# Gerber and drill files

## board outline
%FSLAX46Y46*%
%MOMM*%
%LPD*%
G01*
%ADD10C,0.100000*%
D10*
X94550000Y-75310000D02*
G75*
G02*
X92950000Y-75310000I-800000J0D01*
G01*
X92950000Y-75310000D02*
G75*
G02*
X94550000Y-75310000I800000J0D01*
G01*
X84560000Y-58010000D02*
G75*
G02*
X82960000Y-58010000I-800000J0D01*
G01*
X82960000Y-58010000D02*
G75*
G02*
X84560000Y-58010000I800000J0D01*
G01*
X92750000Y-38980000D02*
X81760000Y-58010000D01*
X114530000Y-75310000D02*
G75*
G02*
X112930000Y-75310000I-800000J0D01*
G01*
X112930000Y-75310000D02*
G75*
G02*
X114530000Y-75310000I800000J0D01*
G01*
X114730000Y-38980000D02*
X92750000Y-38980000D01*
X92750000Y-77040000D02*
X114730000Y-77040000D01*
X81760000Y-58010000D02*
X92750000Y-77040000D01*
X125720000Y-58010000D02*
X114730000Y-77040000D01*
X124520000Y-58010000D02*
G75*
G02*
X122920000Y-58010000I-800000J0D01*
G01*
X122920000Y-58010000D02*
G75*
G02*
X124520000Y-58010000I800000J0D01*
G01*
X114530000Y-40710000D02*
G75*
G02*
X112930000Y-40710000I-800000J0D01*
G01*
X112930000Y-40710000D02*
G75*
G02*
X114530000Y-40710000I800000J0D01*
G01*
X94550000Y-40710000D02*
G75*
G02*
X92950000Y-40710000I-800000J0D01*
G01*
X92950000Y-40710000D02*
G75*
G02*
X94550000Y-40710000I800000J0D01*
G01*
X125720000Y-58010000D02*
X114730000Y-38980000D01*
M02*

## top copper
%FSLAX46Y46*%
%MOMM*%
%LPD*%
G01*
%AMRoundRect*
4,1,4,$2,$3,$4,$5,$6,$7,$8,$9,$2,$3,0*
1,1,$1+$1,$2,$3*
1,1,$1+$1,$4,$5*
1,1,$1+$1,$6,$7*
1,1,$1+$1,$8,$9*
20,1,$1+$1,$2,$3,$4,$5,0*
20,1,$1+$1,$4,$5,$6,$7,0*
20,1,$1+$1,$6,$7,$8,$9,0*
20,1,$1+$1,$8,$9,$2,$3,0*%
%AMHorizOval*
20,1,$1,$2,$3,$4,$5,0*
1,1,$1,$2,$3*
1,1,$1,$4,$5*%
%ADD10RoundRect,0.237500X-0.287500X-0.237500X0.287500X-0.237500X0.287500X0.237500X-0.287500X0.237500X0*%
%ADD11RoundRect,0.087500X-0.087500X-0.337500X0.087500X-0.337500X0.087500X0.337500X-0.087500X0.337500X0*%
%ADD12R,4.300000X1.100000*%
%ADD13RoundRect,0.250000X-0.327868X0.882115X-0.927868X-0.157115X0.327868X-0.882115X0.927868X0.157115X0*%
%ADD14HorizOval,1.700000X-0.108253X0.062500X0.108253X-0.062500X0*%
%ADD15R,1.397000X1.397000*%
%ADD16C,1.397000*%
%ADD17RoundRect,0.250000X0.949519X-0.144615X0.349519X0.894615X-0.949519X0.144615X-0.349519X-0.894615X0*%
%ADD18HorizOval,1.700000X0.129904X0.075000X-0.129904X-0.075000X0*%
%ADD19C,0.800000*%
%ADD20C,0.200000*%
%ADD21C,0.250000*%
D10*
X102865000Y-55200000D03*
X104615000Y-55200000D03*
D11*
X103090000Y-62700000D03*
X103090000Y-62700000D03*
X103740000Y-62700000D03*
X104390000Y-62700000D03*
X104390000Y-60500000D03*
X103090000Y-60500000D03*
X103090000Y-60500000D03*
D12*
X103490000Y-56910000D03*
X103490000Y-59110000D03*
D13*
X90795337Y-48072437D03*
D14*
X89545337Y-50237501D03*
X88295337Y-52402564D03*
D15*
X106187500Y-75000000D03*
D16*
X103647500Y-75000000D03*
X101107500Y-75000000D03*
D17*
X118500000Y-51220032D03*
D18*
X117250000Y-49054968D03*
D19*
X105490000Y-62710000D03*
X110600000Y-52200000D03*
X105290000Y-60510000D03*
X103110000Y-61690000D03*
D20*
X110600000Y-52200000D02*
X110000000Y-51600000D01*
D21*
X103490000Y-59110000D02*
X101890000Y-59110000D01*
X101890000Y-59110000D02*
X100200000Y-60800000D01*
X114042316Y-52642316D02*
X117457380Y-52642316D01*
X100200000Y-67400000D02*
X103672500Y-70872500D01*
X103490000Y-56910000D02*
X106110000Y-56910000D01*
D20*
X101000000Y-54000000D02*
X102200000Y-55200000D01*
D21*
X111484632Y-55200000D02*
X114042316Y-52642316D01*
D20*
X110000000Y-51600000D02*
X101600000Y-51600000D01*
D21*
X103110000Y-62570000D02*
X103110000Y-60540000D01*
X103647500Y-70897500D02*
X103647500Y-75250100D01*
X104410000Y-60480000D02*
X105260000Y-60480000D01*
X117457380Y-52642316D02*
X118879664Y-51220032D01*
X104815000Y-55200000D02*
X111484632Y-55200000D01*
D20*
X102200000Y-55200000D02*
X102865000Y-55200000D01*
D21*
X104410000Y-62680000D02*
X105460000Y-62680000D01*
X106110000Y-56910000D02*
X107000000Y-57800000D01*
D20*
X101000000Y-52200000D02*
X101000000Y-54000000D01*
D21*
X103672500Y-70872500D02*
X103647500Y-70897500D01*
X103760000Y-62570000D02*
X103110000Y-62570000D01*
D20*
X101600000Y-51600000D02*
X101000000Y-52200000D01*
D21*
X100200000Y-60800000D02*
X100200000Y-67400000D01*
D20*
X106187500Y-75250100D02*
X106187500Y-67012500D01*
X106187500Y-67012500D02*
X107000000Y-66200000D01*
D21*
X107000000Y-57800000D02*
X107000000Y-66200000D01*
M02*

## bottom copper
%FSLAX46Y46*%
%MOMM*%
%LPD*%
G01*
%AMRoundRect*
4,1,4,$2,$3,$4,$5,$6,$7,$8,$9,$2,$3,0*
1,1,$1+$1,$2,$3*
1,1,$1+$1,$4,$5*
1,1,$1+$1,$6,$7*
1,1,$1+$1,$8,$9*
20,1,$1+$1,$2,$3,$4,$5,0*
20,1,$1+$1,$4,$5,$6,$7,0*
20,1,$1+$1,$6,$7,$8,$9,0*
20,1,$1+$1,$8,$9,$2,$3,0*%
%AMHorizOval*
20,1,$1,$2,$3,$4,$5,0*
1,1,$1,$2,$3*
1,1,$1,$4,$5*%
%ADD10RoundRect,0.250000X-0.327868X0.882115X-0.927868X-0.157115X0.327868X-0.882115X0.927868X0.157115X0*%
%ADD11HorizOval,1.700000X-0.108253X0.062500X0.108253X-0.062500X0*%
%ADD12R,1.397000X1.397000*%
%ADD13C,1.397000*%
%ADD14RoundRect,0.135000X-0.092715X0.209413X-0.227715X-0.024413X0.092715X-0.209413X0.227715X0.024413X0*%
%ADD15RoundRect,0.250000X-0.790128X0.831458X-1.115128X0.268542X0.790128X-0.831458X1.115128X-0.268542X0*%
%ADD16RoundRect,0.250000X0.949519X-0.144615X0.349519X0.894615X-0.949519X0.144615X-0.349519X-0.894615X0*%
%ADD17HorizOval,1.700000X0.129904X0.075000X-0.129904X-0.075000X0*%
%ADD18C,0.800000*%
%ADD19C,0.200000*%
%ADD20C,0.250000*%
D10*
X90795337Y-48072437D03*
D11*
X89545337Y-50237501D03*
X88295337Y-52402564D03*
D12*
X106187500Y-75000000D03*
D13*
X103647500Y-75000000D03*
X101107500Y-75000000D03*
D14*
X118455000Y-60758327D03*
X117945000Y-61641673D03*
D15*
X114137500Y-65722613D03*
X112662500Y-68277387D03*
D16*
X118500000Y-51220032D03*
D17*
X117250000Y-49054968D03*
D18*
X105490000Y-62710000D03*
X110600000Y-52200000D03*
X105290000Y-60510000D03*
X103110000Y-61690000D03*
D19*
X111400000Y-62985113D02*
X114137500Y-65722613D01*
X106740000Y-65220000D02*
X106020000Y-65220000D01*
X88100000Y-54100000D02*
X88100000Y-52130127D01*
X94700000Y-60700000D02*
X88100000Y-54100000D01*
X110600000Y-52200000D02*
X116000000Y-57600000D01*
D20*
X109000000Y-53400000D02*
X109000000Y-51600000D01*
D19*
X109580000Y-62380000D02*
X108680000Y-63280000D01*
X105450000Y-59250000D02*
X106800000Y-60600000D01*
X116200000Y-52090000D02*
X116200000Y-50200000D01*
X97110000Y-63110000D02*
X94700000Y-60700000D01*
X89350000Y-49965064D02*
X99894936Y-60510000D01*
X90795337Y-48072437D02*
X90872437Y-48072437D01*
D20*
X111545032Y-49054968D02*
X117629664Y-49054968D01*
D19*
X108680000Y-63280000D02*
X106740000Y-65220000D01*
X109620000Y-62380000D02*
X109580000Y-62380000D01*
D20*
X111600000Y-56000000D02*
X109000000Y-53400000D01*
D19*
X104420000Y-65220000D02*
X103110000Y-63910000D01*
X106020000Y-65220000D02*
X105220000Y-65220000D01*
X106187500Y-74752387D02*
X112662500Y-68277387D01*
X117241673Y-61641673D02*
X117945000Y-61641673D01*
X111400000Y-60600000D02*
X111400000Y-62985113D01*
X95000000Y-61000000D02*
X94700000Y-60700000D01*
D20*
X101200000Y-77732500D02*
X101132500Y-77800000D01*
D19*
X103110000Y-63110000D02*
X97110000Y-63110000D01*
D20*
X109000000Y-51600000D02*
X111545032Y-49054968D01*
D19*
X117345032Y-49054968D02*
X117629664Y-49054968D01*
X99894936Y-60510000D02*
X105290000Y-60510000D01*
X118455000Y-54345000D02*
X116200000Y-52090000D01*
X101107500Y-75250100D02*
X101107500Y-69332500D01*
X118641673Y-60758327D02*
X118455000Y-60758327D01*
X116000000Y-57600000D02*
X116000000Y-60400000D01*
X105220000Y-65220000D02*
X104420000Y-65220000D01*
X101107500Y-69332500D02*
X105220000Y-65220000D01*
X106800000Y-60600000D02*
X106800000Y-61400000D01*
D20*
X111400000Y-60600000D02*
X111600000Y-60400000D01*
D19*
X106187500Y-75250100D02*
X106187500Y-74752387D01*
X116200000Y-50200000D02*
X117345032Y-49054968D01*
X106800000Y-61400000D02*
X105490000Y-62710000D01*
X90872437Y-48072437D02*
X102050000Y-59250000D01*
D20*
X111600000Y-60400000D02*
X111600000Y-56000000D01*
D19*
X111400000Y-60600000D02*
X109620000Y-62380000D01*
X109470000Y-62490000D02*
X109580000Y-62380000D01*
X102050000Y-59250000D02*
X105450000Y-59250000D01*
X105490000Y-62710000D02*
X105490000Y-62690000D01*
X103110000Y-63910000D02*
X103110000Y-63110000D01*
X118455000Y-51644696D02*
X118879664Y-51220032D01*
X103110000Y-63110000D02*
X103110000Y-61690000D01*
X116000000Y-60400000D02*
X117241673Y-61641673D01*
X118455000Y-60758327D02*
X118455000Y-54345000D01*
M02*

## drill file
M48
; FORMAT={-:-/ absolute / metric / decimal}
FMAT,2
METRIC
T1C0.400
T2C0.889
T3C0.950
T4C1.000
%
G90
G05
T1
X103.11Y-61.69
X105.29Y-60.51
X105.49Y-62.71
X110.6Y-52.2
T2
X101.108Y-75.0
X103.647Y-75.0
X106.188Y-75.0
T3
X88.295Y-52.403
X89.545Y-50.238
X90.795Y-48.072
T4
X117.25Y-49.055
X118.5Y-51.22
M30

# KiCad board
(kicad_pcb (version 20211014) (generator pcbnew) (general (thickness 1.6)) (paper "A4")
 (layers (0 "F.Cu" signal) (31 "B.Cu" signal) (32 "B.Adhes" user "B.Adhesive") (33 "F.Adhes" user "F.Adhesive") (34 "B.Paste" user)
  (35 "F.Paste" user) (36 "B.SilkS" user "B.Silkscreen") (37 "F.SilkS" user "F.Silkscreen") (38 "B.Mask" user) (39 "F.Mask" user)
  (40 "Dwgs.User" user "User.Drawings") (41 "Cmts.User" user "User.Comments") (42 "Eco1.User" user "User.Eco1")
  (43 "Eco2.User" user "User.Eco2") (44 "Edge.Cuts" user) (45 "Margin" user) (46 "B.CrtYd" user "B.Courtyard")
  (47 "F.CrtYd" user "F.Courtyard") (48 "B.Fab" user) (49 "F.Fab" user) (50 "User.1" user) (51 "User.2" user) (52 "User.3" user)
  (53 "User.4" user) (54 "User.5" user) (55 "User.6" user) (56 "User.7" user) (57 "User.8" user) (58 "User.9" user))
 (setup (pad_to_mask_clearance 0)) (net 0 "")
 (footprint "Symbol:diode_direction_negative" (layer "F.Cu") (at 103.8 52.65)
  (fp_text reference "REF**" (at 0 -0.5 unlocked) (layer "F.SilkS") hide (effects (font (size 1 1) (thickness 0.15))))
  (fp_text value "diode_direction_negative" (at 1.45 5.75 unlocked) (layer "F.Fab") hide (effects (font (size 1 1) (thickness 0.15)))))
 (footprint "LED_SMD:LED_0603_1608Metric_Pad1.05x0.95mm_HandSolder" (layer "F.Cu") (at 103.74 55.2)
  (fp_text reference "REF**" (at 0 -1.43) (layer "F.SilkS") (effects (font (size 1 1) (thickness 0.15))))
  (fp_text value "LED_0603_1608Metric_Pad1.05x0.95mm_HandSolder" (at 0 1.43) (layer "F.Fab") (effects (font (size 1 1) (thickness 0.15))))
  (pad "1" smd roundrect (at -0.875 0) (size 1.05 0.95) (layers "F.Cu" "F.Paste" "F.Mask") (roundrect_rratio 0.25))
  (pad "2" smd roundrect (at 0.875 0) (size 1.05 0.95) (layers "F.Cu" "F.Paste" "F.Mask") (roundrect_rratio 0.25)))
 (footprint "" (layer "F.Cu") (at 103.09 62.7)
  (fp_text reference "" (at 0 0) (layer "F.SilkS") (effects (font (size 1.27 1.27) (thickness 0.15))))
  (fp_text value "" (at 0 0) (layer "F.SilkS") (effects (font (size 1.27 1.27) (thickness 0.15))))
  (pad "1" smd roundrect (at 0 0) (size 0.35 0.85) (layers "F.Cu" "F.Paste" "F.Mask") (roundrect_rratio 0.25)))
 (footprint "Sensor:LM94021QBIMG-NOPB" (layer "F.Cu") (at 103.74 61.6)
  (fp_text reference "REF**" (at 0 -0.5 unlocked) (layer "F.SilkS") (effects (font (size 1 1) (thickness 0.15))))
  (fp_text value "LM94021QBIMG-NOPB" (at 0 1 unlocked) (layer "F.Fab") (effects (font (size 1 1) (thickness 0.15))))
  (pad "1" smd roundrect (at -0.65 1.1) (size 0.35 0.85) (layers "F.Cu" "F.Paste" "F.Mask") (roundrect_rratio 0.25))
  (pad "2" smd roundrect (at 0 1.1) (size 0.35 0.85) (layers "F.Cu" "F.Paste" "F.Mask") (roundrect_rratio 0.25))
  (pad "3" smd roundrect (at 0.65 1.1) (size 0.35 0.85) (layers "F.Cu" "F.Paste" "F.Mask") (roundrect_rratio 0.25))
  (pad "4" smd roundrect (at 0.65 -1.1) (size 0.35 0.85) (layers "F.Cu" "F.Paste" "F.Mask") (roundrect_rratio 0.25))
  (pad "5" smd roundrect (at -0.65 -1.1) (size 0.35 0.85) (layers "F.Cu" "F.Paste" "F.Mask") (roundrect_rratio 0.25)))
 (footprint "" (layer "F.Cu") (at 103.09 60.5)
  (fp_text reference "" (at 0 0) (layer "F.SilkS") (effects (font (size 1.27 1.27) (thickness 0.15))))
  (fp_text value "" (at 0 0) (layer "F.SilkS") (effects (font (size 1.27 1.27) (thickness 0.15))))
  (pad "5" smd roundrect (at 0 0) (size 0.35 0.85) (layers "F.Cu" "F.Paste" "F.Mask") (roundrect_rratio 0.25)))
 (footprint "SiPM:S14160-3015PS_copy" (layer "F.Cu") (at 103.74 58.01)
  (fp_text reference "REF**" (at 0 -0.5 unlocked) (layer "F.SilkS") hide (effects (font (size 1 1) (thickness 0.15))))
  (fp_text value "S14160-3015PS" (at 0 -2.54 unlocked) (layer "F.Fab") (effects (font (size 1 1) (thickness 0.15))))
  (pad "1" smd rect (at -0.25 -1.1) (size 4.3 1.1) (layers "F.Cu" "F.Paste" "F.Mask"))
  (pad "2" smd rect (at -0.25 1.1) (size 4.3 1.1) (layers "F.Cu" "F.Paste" "F.Mask")))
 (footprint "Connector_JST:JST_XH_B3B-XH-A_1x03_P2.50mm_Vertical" (layer "B.Cu") (at 90.795337 48.072437 -120)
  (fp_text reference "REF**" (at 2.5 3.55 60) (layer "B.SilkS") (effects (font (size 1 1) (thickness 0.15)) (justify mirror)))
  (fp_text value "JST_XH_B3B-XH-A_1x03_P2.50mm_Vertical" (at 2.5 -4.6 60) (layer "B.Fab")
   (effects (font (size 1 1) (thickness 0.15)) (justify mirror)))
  (pad "1" thru_hole roundrect (at 0 0 240) (size 1.7 1.95) (drill 0.95) (layers *.Cu *.Mask) (roundrect_rratio 0.1470588235))
  (pad "2" thru_hole oval (at 2.5 0 240) (size 1.7 1.95) (drill 0.95) (layers *.Cu *.Mask))
  (pad "3" thru_hole oval (at 5 0 240) (size 1.7 1.95) (drill 0.95) (layers *.Cu *.Mask)))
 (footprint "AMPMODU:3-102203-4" (layer "B.Cu") (at 106.1875 75 180)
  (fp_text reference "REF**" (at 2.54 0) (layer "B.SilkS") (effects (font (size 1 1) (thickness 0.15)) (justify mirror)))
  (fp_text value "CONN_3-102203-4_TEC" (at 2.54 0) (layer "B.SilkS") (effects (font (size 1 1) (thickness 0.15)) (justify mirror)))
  (pad "1" thru_hole rect locked (at 0 0 180) (size 1.397 1.397) (drill 0.889) (layers *.Cu *.Mask))
  (pad "2" thru_hole circle locked (at 2.54 0 180) (size 1.397 1.397) (drill 0.889) (layers *.Cu *.Mask))
  (pad "3" thru_hole circle locked (at 5.08 0 180) (size 1.397 1.397) (drill 0.889) (layers *.Cu *.Mask)))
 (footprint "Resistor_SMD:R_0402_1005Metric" (layer "B.Cu") (at 118.2 61.2 -120)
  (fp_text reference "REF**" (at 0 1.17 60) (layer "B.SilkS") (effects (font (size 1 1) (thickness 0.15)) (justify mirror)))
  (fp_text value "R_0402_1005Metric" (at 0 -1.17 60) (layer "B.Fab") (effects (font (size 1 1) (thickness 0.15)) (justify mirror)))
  (pad "1" smd roundrect (at -0.51 0 240) (size 0.54 0.64) (layers "B.Cu" "B.Paste" "B.Mask") (roundrect_rratio 0.25))
  (pad "2" smd roundrect (at 0.51 0 240) (size 0.54 0.64) (layers "B.Cu" "B.Paste" "B.Mask") (roundrect_rratio 0.25)))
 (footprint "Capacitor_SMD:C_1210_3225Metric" (layer "B.Cu") (at 113.4 67 -120)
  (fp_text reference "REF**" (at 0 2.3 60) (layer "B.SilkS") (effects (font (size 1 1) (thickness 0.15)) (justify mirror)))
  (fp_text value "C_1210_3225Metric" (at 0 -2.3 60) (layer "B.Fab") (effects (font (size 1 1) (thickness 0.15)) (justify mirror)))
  (pad "1" smd roundrect (at -1.475 0 240) (size 1.15 2.7) (layers "B.Cu" "B.Paste" "B.Mask") (roundrect_rratio 0.2173913043))
  (pad "2" smd roundrect (at 1.475 0 240) (size 1.15 2.7) (layers "B.Cu" "B.Paste" "B.Mask") (roundrect_rratio 0.2173913043)))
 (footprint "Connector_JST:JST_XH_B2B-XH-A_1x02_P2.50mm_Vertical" (layer "B.Cu") (at 118.5 51.220032 120)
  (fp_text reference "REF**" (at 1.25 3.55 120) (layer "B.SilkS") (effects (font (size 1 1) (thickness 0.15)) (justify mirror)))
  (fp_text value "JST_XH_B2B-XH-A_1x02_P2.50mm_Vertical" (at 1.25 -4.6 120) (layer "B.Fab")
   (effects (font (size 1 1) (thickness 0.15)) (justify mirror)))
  (pad "1" thru_hole roundrect (at 0 0 120) (size 1.7 2) (drill 1) (layers *.Cu *.Mask) (roundrect_rratio 0.1470588235))
  (pad "2" thru_hole oval (at 2.5 0 120) (size 1.7 2) (drill 1) (layers *.Cu *.Mask)))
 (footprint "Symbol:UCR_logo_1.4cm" (layer "B.Cu") (at 104.4 43 180)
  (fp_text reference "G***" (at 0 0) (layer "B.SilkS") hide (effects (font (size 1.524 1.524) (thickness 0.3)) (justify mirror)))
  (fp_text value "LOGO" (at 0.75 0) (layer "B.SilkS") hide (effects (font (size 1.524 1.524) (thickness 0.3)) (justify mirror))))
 (gr_circle (center 93.75 75.31) (end 94.55 75.31) (layer "Edge.Cuts") (width 0.1) (fill none))
 (gr_circle (center 83.76 58.01) (end 84.56 58.01) (layer "Edge.Cuts") (width 0.1) (fill none))
 (gr_line (start 92.75 38.98) (end 81.76 58.01) (layer "Edge.Cuts") (width 0.1))
 (gr_circle (center 113.73 75.31) (end 114.53 75.31) (layer "Edge.Cuts") (width 0.1) (fill none))
 (gr_line (start 114.73 38.98) (end 92.75 38.98) (layer "Edge.Cuts") (width 0.1))
 (gr_line (start 92.75 77.04) (end 114.73 77.04) (layer "Edge.Cuts") (width 0.1))
 (gr_line (start 81.76 58.01) (end 92.75 77.04) (layer "Edge.Cuts") (width 0.1))
 (gr_line (start 125.72 58.01) (end 114.73 77.04) (layer "Edge.Cuts") (width 0.1))
 (gr_circle (center 123.72 58.01) (end 124.52 58.01) (layer "Edge.Cuts") (width 0.1) (fill none))
 (gr_circle (center 113.73 40.71) (end 114.53 40.71) (layer "Edge.Cuts") (width 0.1) (fill none))
 (gr_circle (center 93.75 40.71) (end 94.55 40.71) (layer "Edge.Cuts") (width 0.1) (fill none))
 (gr_line (start 125.72 58.01) (end 114.73 38.98) (layer "Edge.Cuts") (width 0.1))
 (segment (start 110.6 52.2) (end 110 51.6) (width 0.2) (layer "F.Cu") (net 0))
 (segment (start 103.49 59.11) (end 101.89 59.11) (width 0.25) (layer "F.Cu") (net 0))
 (segment (start 101.89 59.11) (end 100.2 60.8) (width 0.25) (layer "F.Cu") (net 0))
 (segment (start 114.042316 52.642316) (end 117.45738 52.642316) (width 0.25) (layer "F.Cu") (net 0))
 (segment (start 100.2 67.4) (end 103.6725 70.8725) (width 0.25) (layer "F.Cu") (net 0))
 (segment (start 103.49 56.91) (end 106.11 56.91) (width 0.25) (layer "F.Cu") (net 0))
 (segment (start 101 54) (end 102.2 55.2) (width 0.2) (layer "F.Cu") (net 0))
 (segment (start 111.484632 55.2) (end 114.042316 52.642316) (width 0.25) (layer "F.Cu") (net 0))
 (segment (start 110 51.6) (end 101.6 51.6) (width 0.2) (layer "F.Cu") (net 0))
 (segment (start 103.11 62.57) (end 103.11 60.54) (width 0.25) (layer "F.Cu") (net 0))
 (segment (start 103.6475 70.8975) (end 103.6475 75.2501) (width 0.25) (layer "F.Cu") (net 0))
 (segment (start 104.41 60.48) (end 105.26 60.48) (width 0.25) (layer "F.Cu") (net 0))
 (segment (start 117.45738 52.642316) (end 118.879664 51.220032) (width 0.25) (layer "F.Cu") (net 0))
 (segment (start 104.815 55.2) (end 111.484632 55.2) (width 0.25) (layer "F.Cu") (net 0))
 (segment (start 102.2 55.2) (end 102.865 55.2) (width 0.2) (layer "F.Cu") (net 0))
 (segment (start 104.41 62.68) (end 105.46 62.68) (width 0.25) (layer "F.Cu") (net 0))
 (segment (start 106.11 56.91) (end 107 57.8) (width 0.25) (layer "F.Cu") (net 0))
 (segment (start 101 52.2) (end 101 54) (width 0.2) (layer "F.Cu") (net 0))
 (segment (start 103.6725 70.8725) (end 103.6475 70.8975) (width 0.25) (layer "F.Cu") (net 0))
 (segment (start 103.76 62.57) (end 103.11 62.57) (width 0.25) (layer "F.Cu") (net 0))
 (segment (start 101.6 51.6) (end 101 52.2) (width 0.2) (layer "F.Cu") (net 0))
 (segment (start 100.2 60.8) (end 100.2 67.4) (width 0.25) (layer "F.Cu") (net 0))
 (segment (start 106.1875 75.2501) (end 106.1875 67.0125) (width 0.2) (layer "F.Cu") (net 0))
 (segment (start 106.1875 67.0125) (end 107 66.2) (width 0.2) (layer "F.Cu") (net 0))
 (segment (start 107 57.8) (end 107 66.2) (width 0.25) (layer "F.Cu") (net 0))
 (via (at 105.49 62.71) (size 0.8) (drill 0.4) (layers "F.Cu" "B.Cu") (free) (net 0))
 (via (at 110.6 52.2) (size 0.8) (drill 0.4) (layers "F.Cu" "B.Cu") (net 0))
 (via (at 105.29 60.51) (size 0.8) (drill 0.4) (layers "F.Cu" "B.Cu") (free) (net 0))
 (via (at 103.11 61.69) (size 0.8) (drill 0.4) (layers "F.Cu" "B.Cu") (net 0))
 (segment (start 111.4 62.985113) (end 114.1375 65.722613) (width 0.2) (layer "B.Cu") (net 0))
 (segment (start 106.74 65.22) (end 106.02 65.22) (width 0.2) (layer "B.Cu") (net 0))
 (segment (start 88.1 54.1) (end 88.1 52.130127) (width 0.2) (layer "B.Cu") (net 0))
 (segment (start 94.7 60.7) (end 88.1 54.1) (width 0.2) (layer "B.Cu") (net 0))
 (segment (start 110.6 52.2) (end 116 57.6) (width 0.2) (layer "B.Cu") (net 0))
 (segment (start 109 53.4) (end 109 51.6) (width 0.25) (layer "B.Cu") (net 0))
 (segment (start 109.58 62.38) (end 108.68 63.28) (width 0.2) (layer "B.Cu") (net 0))
 (segment (start 105.45 59.25) (end 106.8 60.6) (width 0.2) (layer "B.Cu") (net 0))
 (segment (start 116.2 52.09) (end 116.2 50.2) (width 0.2) (layer "B.Cu") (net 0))
 (segment (start 97.11 63.11) (end 94.7 60.7) (width 0.2) (layer "B.Cu") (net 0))
 (segment (start 89.35 49.965064) (end 99.894936 60.51) (width 0.2) (layer "B.Cu") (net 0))
 (segment (start 90.795337 48.072437) (end 90.872437 48.072437) (width 0.2) (layer "B.Cu") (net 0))
 (segment (start 111.545032 49.054968) (end 117.629664 49.054968) (width 0.25) (layer "B.Cu") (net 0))
 (segment (start 108.68 63.28) (end 106.74 65.22) (width 0.2) (layer "B.Cu") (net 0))
 (segment (start 109.62 62.38) (end 109.58 62.38) (width 0.2) (layer "B.Cu") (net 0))
 (segment (start 111.6 56) (end 109 53.4) (width 0.25) (layer "B.Cu") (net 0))
 (segment (start 104.42 65.22) (end 103.11 63.91) (width 0.2) (layer "B.Cu") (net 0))
 (segment (start 106.02 65.22) (end 105.22 65.22) (width 0.2) (layer "B.Cu") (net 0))
 (segment (start 106.1875 74.752387) (end 112.6625 68.277387) (width 0.2) (layer "B.Cu") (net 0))
 (segment (start 117.241673 61.641673) (end 117.945 61.641673) (width 0.2) (layer "B.Cu") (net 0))
 (segment (start 111.4 60.6) (end 111.4 62.985113) (width 0.2) (layer "B.Cu") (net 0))
 (segment (start 95 61) (end 94.7 60.7) (width 0.2) (layer "B.Cu") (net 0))
 (segment (start 101.2 77.7325) (end 101.1325 77.8) (width 0.25) (layer "B.Cu") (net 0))
 (segment (start 103.11 63.11) (end 97.11 63.11) (width 0.2) (layer "B.Cu") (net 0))
 (segment (start 109 51.6) (end 111.545032 49.054968) (width 0.25) (layer "B.Cu") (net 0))
 (segment (start 117.345032 49.054968) (end 117.629664 49.054968) (width 0.2) (layer "B.Cu") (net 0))
 (segment (start 99.894936 60.51) (end 105.29 60.51) (width 0.2) (layer "B.Cu") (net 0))
 (segment (start 118.455 54.345) (end 116.2 52.09) (width 0.2) (layer "B.Cu") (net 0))
 (segment (start 101.1075 75.2501) (end 101.1075 69.3325) (width 0.2) (layer "B.Cu") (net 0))
 (segment (start 118.641673 60.758327) (end 118.455 60.758327) (width 0.2) (layer "B.Cu") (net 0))
 (segment (start 116 57.6) (end 116 60.4) (width 0.2) (layer "B.Cu") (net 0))
 (segment (start 105.22 65.22) (end 104.42 65.22) (width 0.2) (layer "B.Cu") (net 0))
 (segment (start 101.1075 69.3325) (end 105.22 65.22) (width 0.2) (layer "B.Cu") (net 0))
 (segment (start 106.8 60.6) (end 106.8 61.4) (width 0.2) (layer "B.Cu") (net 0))
 (segment (start 111.4 60.6) (end 111.6 60.4) (width 0.25) (layer "B.Cu") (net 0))
 (segment (start 106.1875 75.2501) (end 106.1875 74.752387) (width 0.2) (layer "B.Cu") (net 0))
 (segment (start 116.2 50.2) (end 117.345032 49.054968) (width 0.2) (layer "B.Cu") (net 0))
 (segment (start 106.8 61.4) (end 105.49 62.71) (width 0.2) (layer "B.Cu") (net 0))
 (segment (start 90.872437 48.072437) (end 102.05 59.25) (width 0.2) (layer "B.Cu") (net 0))
 (segment (start 111.6 60.4) (end 111.6 56) (width 0.25) (layer "B.Cu") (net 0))
 (segment (start 111.4 60.6) (end 109.62 62.38) (width 0.2) (layer "B.Cu") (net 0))
 (segment (start 109.47 62.49) (end 109.58 62.38) (width 0.2) (layer "B.Cu") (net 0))
 (segment (start 102.05 59.25) (end 105.45 59.25) (width 0.2) (layer "B.Cu") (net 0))
 (segment (start 105.49 62.71) (end 105.49 62.69) (width 0.2) (layer "B.Cu") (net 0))
 (segment (start 103.11 63.91) (end 103.11 63.11) (width 0.2) (layer "B.Cu") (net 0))
 (segment (start 118.455 51.644696) (end 118.879664 51.220032) (width 0.2) (layer "B.Cu") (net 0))
 (segment (start 103.11 63.11) (end 103.11 61.69) (width 0.2) (layer "B.Cu") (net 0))
 (segment (start 116 60.4) (end 117.241673 61.641673) (width 0.2) (layer "B.Cu") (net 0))
 (segment (start 118.455 60.758327) (end 118.455 54.345) (width 0.2) (layer "B.Cu") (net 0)))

